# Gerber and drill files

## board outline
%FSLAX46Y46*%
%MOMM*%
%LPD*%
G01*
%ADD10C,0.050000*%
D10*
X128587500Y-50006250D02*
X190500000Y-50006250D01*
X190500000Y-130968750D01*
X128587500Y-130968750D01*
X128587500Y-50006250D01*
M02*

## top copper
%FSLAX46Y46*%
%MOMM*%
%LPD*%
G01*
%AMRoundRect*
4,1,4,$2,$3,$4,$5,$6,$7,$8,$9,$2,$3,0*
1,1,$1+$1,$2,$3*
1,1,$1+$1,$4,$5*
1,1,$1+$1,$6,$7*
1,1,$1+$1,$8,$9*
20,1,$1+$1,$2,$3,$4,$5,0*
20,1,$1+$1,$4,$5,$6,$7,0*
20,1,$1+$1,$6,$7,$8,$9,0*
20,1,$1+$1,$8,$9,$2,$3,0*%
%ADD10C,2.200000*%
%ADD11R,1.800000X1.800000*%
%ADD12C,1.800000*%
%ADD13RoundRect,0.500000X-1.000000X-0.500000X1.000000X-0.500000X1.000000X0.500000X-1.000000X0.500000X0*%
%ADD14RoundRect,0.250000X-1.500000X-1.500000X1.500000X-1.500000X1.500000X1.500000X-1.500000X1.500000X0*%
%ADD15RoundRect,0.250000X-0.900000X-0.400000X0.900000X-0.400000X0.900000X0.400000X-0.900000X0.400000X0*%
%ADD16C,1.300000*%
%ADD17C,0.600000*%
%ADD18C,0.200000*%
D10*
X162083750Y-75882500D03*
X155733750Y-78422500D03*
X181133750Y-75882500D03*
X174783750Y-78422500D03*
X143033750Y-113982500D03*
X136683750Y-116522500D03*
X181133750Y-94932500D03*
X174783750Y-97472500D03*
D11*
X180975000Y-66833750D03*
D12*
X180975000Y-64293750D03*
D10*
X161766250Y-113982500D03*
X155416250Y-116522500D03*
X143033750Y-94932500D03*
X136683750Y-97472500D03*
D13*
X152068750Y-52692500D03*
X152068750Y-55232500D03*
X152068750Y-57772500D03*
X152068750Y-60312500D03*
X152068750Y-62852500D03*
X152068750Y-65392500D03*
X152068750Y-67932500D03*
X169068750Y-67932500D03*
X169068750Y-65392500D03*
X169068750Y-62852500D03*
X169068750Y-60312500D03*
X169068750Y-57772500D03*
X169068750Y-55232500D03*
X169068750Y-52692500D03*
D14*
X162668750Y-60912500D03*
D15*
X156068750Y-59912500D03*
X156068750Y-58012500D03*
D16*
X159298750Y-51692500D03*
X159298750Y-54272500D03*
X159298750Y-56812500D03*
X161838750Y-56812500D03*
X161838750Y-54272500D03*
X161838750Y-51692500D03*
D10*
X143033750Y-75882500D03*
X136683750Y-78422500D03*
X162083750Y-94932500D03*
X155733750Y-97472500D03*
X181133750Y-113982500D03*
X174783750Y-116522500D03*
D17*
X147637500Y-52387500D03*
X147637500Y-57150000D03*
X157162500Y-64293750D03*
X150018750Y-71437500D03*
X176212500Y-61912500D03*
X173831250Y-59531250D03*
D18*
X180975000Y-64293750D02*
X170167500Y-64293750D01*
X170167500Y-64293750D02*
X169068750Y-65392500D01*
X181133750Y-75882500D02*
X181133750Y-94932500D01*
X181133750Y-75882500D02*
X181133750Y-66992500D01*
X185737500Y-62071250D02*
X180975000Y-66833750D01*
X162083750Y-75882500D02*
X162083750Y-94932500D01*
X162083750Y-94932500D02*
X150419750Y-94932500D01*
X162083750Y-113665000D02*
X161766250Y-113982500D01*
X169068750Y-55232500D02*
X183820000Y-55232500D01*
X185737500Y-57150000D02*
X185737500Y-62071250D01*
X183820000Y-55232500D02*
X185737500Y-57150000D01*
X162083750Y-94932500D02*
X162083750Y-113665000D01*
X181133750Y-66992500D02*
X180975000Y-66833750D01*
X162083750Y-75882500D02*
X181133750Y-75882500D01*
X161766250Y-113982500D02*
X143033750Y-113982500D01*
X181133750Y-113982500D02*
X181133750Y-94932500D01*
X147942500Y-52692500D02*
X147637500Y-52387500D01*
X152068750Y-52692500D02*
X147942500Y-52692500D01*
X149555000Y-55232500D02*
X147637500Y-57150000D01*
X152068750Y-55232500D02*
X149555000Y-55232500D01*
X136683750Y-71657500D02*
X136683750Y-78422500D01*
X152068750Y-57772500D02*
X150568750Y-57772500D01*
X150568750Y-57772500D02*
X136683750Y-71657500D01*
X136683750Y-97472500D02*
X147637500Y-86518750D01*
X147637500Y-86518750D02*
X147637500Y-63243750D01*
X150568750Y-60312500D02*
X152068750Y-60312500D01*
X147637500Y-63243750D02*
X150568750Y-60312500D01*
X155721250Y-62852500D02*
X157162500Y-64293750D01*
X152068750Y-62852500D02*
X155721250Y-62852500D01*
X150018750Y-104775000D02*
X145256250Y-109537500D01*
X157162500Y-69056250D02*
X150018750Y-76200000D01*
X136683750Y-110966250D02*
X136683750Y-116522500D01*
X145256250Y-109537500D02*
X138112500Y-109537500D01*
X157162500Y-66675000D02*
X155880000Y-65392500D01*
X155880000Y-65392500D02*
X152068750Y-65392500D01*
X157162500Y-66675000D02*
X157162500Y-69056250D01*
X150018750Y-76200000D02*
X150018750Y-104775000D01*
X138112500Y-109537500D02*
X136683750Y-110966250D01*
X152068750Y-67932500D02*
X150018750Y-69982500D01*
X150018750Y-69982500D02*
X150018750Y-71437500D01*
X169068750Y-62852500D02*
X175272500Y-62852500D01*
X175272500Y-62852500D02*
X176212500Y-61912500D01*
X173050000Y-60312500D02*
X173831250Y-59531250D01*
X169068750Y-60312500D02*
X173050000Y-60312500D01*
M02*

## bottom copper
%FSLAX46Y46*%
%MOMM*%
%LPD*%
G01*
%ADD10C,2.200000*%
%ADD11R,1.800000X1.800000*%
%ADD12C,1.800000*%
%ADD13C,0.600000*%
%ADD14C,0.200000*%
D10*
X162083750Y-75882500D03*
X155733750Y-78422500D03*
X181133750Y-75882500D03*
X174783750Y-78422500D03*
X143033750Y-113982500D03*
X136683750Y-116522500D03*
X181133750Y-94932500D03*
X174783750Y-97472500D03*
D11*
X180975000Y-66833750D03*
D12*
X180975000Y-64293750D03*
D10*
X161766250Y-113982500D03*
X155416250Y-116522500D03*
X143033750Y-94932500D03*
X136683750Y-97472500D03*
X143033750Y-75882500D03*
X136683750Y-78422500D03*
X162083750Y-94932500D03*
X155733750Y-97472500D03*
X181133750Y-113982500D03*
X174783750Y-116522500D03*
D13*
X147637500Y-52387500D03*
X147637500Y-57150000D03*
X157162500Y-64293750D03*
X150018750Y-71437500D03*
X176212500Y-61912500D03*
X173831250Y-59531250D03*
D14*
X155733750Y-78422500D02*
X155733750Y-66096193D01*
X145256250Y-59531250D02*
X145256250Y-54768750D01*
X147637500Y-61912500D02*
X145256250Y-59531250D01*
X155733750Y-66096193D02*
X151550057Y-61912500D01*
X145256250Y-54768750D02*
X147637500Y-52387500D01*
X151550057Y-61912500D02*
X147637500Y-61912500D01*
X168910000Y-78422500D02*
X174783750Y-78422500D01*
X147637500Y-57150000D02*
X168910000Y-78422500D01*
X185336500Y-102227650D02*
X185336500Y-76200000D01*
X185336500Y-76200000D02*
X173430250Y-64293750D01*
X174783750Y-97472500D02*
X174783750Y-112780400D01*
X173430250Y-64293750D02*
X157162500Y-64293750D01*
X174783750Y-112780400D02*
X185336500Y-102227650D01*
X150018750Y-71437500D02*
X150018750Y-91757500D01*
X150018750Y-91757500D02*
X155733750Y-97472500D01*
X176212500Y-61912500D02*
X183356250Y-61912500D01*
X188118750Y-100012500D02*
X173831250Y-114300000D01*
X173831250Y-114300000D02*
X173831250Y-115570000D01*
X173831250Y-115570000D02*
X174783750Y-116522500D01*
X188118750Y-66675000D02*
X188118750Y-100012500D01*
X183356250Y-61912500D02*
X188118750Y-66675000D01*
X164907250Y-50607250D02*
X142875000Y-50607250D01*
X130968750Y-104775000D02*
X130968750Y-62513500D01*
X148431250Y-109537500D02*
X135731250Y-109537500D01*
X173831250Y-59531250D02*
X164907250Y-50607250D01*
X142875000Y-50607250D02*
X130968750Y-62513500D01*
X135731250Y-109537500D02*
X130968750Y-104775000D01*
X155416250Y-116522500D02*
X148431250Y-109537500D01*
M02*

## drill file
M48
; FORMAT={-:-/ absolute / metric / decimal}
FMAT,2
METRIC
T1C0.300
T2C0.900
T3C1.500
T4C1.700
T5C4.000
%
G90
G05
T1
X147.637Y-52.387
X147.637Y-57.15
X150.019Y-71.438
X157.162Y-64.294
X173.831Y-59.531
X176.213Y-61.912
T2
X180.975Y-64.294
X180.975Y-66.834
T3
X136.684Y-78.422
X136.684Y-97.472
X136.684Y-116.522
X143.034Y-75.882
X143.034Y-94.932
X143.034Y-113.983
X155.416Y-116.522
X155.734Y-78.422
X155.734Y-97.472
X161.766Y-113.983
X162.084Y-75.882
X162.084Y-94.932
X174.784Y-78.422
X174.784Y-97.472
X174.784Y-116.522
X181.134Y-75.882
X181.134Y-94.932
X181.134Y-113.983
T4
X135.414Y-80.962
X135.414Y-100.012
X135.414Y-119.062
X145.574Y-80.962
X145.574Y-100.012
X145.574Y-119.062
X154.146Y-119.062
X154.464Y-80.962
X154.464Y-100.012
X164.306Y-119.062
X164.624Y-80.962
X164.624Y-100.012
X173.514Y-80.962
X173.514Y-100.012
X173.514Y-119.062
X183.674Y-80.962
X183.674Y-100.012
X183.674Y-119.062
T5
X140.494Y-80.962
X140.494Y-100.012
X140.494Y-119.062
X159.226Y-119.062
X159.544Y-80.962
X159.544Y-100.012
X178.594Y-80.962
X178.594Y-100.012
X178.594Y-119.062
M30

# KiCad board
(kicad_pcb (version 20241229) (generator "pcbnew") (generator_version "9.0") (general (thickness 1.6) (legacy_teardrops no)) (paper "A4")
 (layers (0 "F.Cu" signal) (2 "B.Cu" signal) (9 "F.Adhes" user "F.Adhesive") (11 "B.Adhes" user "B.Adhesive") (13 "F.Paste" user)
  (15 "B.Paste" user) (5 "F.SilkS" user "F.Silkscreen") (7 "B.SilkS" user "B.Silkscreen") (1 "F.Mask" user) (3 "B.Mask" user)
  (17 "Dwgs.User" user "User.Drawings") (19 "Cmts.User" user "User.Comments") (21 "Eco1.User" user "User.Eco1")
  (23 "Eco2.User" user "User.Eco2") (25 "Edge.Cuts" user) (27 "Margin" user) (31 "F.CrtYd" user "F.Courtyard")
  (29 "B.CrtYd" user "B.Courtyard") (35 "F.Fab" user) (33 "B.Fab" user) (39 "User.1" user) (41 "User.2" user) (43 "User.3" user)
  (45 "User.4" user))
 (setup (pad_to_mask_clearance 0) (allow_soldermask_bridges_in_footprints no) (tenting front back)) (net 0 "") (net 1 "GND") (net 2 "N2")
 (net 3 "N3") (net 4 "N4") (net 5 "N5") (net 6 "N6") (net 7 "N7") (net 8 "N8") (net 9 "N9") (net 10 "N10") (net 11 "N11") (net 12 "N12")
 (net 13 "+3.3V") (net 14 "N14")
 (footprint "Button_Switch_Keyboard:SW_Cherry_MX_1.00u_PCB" (layer "F.Cu") (at 162.08375 75.8825)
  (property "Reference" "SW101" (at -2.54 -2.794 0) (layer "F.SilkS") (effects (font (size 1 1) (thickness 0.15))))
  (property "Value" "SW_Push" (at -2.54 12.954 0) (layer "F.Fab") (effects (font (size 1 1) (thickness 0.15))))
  (pad "" np_thru_hole circle (at -7.62 5.08) (size 1.7 1.7) (drill 1.7) (layers "*.Cu" "*.Mask"))
  (pad "" np_thru_hole circle (at -2.54 5.08) (size 4 4) (drill 4) (layers "*.Cu" "*.Mask"))
  (pad "" np_thru_hole circle (at 2.54 5.08) (size 1.7 1.7) (drill 1.7) (layers "*.Cu" "*.Mask"))
  (pad "1" thru_hole circle (at 0 0) (size 2.2 2.2) (drill 1.5) (layers "*.Cu" "*.Mask") (remove_unused_layers no) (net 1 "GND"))
  (pad "2" thru_hole circle (at -6.35 2.54) (size 2.2 2.2) (drill 1.5) (layers "*.Cu" "*.Mask") (remove_unused_layers no) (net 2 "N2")))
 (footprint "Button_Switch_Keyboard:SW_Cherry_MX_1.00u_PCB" (layer "F.Cu") (at 181.13375 75.8825)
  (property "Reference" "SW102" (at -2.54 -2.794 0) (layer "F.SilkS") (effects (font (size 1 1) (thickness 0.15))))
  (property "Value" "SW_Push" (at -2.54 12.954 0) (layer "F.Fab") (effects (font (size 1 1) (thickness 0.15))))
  (pad "" np_thru_hole circle (at -7.62 5.08) (size 1.7 1.7) (drill 1.7) (layers "*.Cu" "*.Mask"))
  (pad "" np_thru_hole circle (at -2.54 5.08) (size 4 4) (drill 4) (layers "*.Cu" "*.Mask"))
  (pad "" np_thru_hole circle (at 2.54 5.08) (size 1.7 1.7) (drill 1.7) (layers "*.Cu" "*.Mask"))
  (pad "1" thru_hole circle (at 0 0) (size 2.2 2.2) (drill 1.5) (layers "*.Cu" "*.Mask") (remove_unused_layers no) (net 1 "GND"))
  (pad "2" thru_hole circle (at -6.35 2.54) (size 2.2 2.2) (drill 1.5) (layers "*.Cu" "*.Mask") (remove_unused_layers no) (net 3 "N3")))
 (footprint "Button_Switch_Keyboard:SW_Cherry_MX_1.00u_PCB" (layer "F.Cu") (at 143.03375 113.9825)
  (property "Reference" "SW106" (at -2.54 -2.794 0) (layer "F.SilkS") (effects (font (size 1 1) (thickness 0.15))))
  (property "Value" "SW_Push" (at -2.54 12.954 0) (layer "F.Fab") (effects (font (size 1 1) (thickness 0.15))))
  (pad "" np_thru_hole circle (at -7.62 5.08) (size 1.7 1.7) (drill 1.7) (layers "*.Cu" "*.Mask"))
  (pad "" np_thru_hole circle (at -2.54 5.08) (size 4 4) (drill 4) (layers "*.Cu" "*.Mask"))
  (pad "" np_thru_hole circle (at 2.54 5.08) (size 1.7 1.7) (drill 1.7) (layers "*.Cu" "*.Mask"))
  (pad "1" thru_hole circle (at 0 0) (size 2.2 2.2) (drill 1.5) (layers "*.Cu" "*.Mask") (remove_unused_layers no) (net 1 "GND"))
  (pad "2" thru_hole circle (at -6.35 2.54) (size 2.2 2.2) (drill 1.5) (layers "*.Cu" "*.Mask") (remove_unused_layers no) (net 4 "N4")))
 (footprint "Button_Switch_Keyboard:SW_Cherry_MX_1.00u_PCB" (layer "F.Cu") (at 181.13375 94.9325)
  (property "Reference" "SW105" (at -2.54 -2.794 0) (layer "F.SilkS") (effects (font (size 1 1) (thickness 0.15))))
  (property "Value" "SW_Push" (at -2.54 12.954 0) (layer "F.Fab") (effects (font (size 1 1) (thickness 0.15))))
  (pad "" np_thru_hole circle (at -7.62 5.08) (size 1.7 1.7) (drill 1.7) (layers "*.Cu" "*.Mask"))
  (pad "" np_thru_hole circle (at -2.54 5.08) (size 4 4) (drill 4) (layers "*.Cu" "*.Mask"))
  (pad "" np_thru_hole circle (at 2.54 5.08) (size 1.7 1.7) (drill 1.7) (layers "*.Cu" "*.Mask"))
  (pad "1" thru_hole circle (at 0 0) (size 2.2 2.2) (drill 1.5) (layers "*.Cu" "*.Mask") (remove_unused_layers no) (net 1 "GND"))
  (pad "2" thru_hole circle (at -6.35 2.54) (size 2.2 2.2) (drill 1.5) (layers "*.Cu" "*.Mask") (remove_unused_layers no) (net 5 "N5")))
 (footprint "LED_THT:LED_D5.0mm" (layer "F.Cu") (at 180.975 66.83375 90)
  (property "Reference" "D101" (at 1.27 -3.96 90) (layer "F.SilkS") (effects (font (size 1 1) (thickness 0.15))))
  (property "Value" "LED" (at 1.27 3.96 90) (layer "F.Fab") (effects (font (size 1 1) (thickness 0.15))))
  (pad "1" thru_hole rect (at 0 0 90) (size 1.8 1.8) (drill 0.9) (layers "*.Cu" "*.Mask") (remove_unused_layers no) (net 1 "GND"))
  (pad "2" thru_hole circle (at 2.54 0 90) (size 1.8 1.8) (drill 0.9) (layers "*.Cu" "*.Mask") (remove_unused_layers no) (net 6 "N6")))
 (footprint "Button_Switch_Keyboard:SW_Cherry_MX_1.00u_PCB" (layer "F.Cu") (at 161.76625 113.9825)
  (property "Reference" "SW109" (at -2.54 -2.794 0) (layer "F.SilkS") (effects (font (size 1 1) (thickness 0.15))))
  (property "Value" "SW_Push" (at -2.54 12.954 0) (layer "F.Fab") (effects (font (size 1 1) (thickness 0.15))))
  (pad "" np_thru_hole circle (at -7.62 5.08) (size 1.7 1.7) (drill 1.7) (layers "*.Cu" "*.Mask"))
  (pad "" np_thru_hole circle (at -2.54 5.08) (size 4 4) (drill 4) (layers "*.Cu" "*.Mask"))
  (pad "" np_thru_hole circle (at 2.54 5.08) (size 1.7 1.7) (drill 1.7) (layers "*.Cu" "*.Mask"))
  (pad "1" thru_hole circle (at 0 0) (size 2.2 2.2) (drill 1.5) (layers "*.Cu" "*.Mask") (remove_unused_layers no) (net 1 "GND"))
  (pad "2" thru_hole circle (at -6.35 2.54) (size 2.2 2.2) (drill 1.5) (layers "*.Cu" "*.Mask") (remove_unused_layers no) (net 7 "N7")))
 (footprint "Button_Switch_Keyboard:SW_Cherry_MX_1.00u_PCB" (layer "F.Cu") (at 143.03375 94.9325)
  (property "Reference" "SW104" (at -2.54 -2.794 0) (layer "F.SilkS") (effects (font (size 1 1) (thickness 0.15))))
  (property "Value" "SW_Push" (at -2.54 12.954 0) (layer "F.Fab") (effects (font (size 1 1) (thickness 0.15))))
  (pad "" np_thru_hole circle (at -7.62 5.08) (size 1.7 1.7) (drill 1.7) (layers "*.Cu" "*.Mask"))
  (pad "" np_thru_hole circle (at -2.54 5.08) (size 4 4) (drill 4) (layers "*.Cu" "*.Mask"))
  (pad "" np_thru_hole circle (at 2.54 5.08) (size 1.7 1.7) (drill 1.7) (layers "*.Cu" "*.Mask"))
  (pad "1" thru_hole circle (at 0 0) (size 2.2 2.2) (drill 1.5) (layers "*.Cu" "*.Mask") (remove_unused_layers no) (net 1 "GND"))
  (pad "2" thru_hole circle (at -6.35 2.54) (size 2.2 2.2) (drill 1.5) (layers "*.Cu" "*.Mask") (remove_unused_layers no) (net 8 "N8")))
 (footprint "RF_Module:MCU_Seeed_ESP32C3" (layer "F.Cu") (at 160.56875 60.3125)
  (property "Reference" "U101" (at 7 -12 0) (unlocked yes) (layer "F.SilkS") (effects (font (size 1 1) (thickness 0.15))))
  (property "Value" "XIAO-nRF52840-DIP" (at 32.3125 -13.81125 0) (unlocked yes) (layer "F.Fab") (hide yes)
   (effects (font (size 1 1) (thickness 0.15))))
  (pad "" smd roundrect (at 1.1 -0.4) (size 1.5 1.5) (layers "F.Paste") (roundrect_rratio 0.1666666667))
  (pad "" smd roundrect (at 1.1 1.6) (size 1.5 1.5) (layers "F.Paste") (roundrect_rratio 0.1666666667))
  (pad "" smd roundrect (at 3.1 -0.4) (size 1.5 1.5) (layers "F.Paste") (roundrect_rratio 0.1666666667))
  (pad "" smd roundrect (at 3.1 1.6) (size 1.5 1.5) (layers "F.Paste") (roundrect_rratio 0.1666666667))
  (pad "1" smd roundrect (at -8.5 -7.62) (size 3 2) (layers "F.Cu" "F.Mask" "F.Paste") (roundrect_rratio 0.25) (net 2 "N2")
   (thermal_bridge_angle 45))
  (pad "2" smd roundrect (at -8.5 -5.08) (size 3 2) (layers "F.Cu" "F.Mask" "F.Paste") (roundrect_rratio 0.25) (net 3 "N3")
   (thermal_bridge_angle 45))
  (pad "3" smd roundrect (at -8.5 -2.54) (size 3 2) (layers "F.Cu" "F.Mask" "F.Paste") (roundrect_rratio 0.25) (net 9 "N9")
   (thermal_bridge_angle 45))
  (pad "4" smd roundrect (at -8.5 0) (size 3 2) (layers "F.Cu" "F.Mask" "F.Paste") (roundrect_rratio 0.25) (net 8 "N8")
   (thermal_bridge_angle 45))
  (pad "5" smd roundrect (at -8.5 2.54) (size 3 2) (layers "F.Cu" "F.Mask" "F.Paste") (roundrect_rratio 0.25) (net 5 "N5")
   (thermal_bridge_angle 45))
  (pad "6" smd roundrect (at -8.5 5.08) (size 3 2) (layers "F.Cu" "F.Mask" "F.Paste") (roundrect_rratio 0.25) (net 4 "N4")
   (thermal_bridge_angle 45))
  (pad "7" smd roundrect (at -8.5 7.62) (size 3 2) (layers "F.Cu" "F.Mask" "F.Paste") (roundrect_rratio 0.25) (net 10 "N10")
   (thermal_bridge_angle 45))
  (pad "8" smd roundrect (at 8.5 7.62) (size 3 2) (layers "F.Cu" "F.Mask" "F.Paste") (roundrect_rratio 0.25) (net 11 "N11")
   (thermal_bridge_angle 45))
  (pad "9" smd roundrect (at 8.5 5.08) (size 3 2) (layers "F.Cu" "F.Mask" "F.Paste") (roundrect_rratio 0.25) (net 6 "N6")
   (thermal_bridge_angle 45))
  (pad "10" smd roundrect (at 8.5 2.54) (size 3 2) (layers "F.Cu" "F.Mask" "F.Paste") (roundrect_rratio 0.25) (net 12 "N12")
   (thermal_bridge_angle 45))
  (pad "11" smd roundrect (at 8.5 0) (size 3 2) (layers "F.Cu" "F.Mask" "F.Paste") (roundrect_rratio 0.25) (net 7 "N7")
   (thermal_bridge_angle 45))
  (pad "12" smd roundrect (at 8.5 -2.54) (size 3 2) (layers "F.Cu" "F.Mask" "F.Paste") (roundrect_rratio 0.25) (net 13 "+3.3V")
   (thermal_bridge_angle 45))
  (pad "13" smd roundrect (at 8.5 -5.08) (size 3 2) (layers "F.Cu" "F.Mask" "F.Paste") (roundrect_rratio 0.25) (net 1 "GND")
   (thermal_bridge_angle 45))
  (pad "14" smd roundrect (at 8.5 -7.62) (size 3 2) (layers "F.Cu" "F.Mask" "F.Paste") (roundrect_rratio 0.25) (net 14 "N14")
   (thermal_bridge_angle 45))
  (pad "15" smd roundrect (at 2.1 0.6) (size 3.5 3.5) (layers "F.Cu" "F.Mask") (roundrect_rratio 0.07142857143))
  (pad "16" smd roundrect (at -4.5 -0.4) (size 2.3 1.3) (layers "F.Cu" "F.Mask" "F.Paste") (roundrect_rratio 0.1923076923))
  (pad "17" smd roundrect (at -4.5 -2.3) (size 2.3 1.3) (layers "F.Cu" "F.Mask" "F.Paste") (roundrect_rratio 0.1923076923))
  (pad "18" smd circle (at -1.27 -8.62) (size 1.3 1.3) (layers "F.Cu" "F.Mask" "F.Paste"))
  (pad "19" smd circle (at -1.27 -6.04) (size 1.3 1.3) (layers "F.Cu" "F.Mask" "F.Paste"))
  (pad "20" smd circle (at -1.27 -3.5) (size 1.3 1.3) (layers "F.Cu" "F.Mask" "F.Paste"))
  (pad "21" smd circle (at 1.27 -3.5) (size 1.3 1.3) (layers "F.Cu" "F.Mask" "F.Paste"))
  (pad "22" smd circle (at 1.27 -6.04) (size 1.3 1.3) (layers "F.Cu" "F.Mask" "F.Paste"))
  (pad "23" smd circle (at 1.27 -8.62) (size 1.3 1.3) (layers "F.Cu" "F.Mask" "F.Paste")))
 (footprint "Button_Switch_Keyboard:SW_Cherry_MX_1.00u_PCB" (layer "F.Cu") (at 143.03375 75.8825)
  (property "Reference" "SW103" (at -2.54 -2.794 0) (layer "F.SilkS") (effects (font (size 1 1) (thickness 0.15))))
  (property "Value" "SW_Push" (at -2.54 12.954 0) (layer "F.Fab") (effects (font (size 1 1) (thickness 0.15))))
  (pad "" np_thru_hole circle (at -7.62 5.08) (size 1.7 1.7) (drill 1.7) (layers "*.Cu" "*.Mask"))
  (pad "" np_thru_hole circle (at -2.54 5.08) (size 4 4) (drill 4) (layers "*.Cu" "*.Mask"))
  (pad "" np_thru_hole circle (at 2.54 5.08) (size 1.7 1.7) (drill 1.7) (layers "*.Cu" "*.Mask"))
  (pad "1" thru_hole circle (at 0 0) (size 2.2 2.2) (drill 1.5) (layers "*.Cu" "*.Mask") (remove_unused_layers no) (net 1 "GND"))
  (pad "2" thru_hole circle (at -6.35 2.54) (size 2.2 2.2) (drill 1.5) (layers "*.Cu" "*.Mask") (remove_unused_layers no) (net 9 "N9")))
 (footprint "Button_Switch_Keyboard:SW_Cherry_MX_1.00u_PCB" (layer "F.Cu") (at 162.08375 94.9325)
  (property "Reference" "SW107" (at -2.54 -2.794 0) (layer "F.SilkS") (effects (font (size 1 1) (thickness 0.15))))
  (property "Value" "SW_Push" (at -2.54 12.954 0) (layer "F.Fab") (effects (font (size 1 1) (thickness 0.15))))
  (pad "" np_thru_hole circle (at -7.62 5.08) (size 1.7 1.7) (drill 1.7) (layers "*.Cu" "*.Mask"))
  (pad "" np_thru_hole circle (at -2.54 5.08) (size 4 4) (drill 4) (layers "*.Cu" "*.Mask"))
  (pad "" np_thru_hole circle (at 2.54 5.08) (size 1.7 1.7) (drill 1.7) (layers "*.Cu" "*.Mask"))
  (pad "1" thru_hole circle (at 0 0) (size 2.2 2.2) (drill 1.5) (layers "*.Cu" "*.Mask") (remove_unused_layers no) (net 1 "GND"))
  (pad "2" thru_hole circle (at -6.35 2.54) (size 2.2 2.2) (drill 1.5) (layers "*.Cu" "*.Mask") (remove_unused_layers no) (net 10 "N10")))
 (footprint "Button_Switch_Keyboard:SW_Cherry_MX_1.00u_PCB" (layer "F.Cu") (at 181.13375 113.9825)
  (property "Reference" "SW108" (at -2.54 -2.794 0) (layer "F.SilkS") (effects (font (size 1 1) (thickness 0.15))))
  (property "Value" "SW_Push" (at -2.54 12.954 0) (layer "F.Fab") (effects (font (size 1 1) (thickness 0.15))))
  (pad "" np_thru_hole circle (at -7.62 5.08) (size 1.7 1.7) (drill 1.7) (layers "*.Cu" "*.Mask"))
  (pad "" np_thru_hole circle (at -2.54 5.08) (size 4 4) (drill 4) (layers "*.Cu" "*.Mask"))
  (pad "" np_thru_hole circle (at 2.54 5.08) (size 1.7 1.7) (drill 1.7) (layers "*.Cu" "*.Mask"))
  (pad "1" thru_hole circle (at 0 0) (size 2.2 2.2) (drill 1.5) (layers "*.Cu" "*.Mask") (remove_unused_layers no) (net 1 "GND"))
  (pad "2" thru_hole circle (at -6.35 2.54) (size 2.2 2.2) (drill 1.5) (layers "*.Cu" "*.Mask") (remove_unused_layers no) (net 12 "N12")))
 (gr_rect (start 128.5875 50.00625) (end 190.5 130.96875) (stroke (width 0.05) (type default)) (fill no) (layer "Edge.Cuts"))
 (segment (start 180.975 64.29375) (end 170.1675 64.29375) (width 0.2) (layer "F.Cu") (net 6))
 (segment (start 170.1675 64.29375) (end 169.06875 65.3925) (width 0.2) (layer "F.Cu") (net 6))
 (segment (start 181.13375 75.8825) (end 181.13375 94.9325) (width 0.2) (layer "F.Cu") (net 1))
 (segment (start 181.13375 75.8825) (end 181.13375 66.9925) (width 0.2) (layer "F.Cu") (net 1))
 (segment (start 185.7375 62.07125) (end 180.975 66.83375) (width 0.2) (layer "F.Cu") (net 1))
 (segment (start 162.08375 75.8825) (end 162.08375 94.9325) (width 0.2) (layer "F.Cu") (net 1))
 (segment (start 162.08375 94.9325) (end 150.41975 94.9325) (width 0.2) (layer "F.Cu") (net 1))
 (segment (start 162.08375 113.665) (end 161.76625 113.9825) (width 0.2) (layer "F.Cu") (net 1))
 (segment (start 169.06875 55.2325) (end 183.82 55.2325) (width 0.2) (layer "F.Cu") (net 1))
 (segment (start 185.7375 57.15) (end 185.7375 62.07125) (width 0.2) (layer "F.Cu") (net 1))
 (segment (start 183.82 55.2325) (end 185.7375 57.15) (width 0.2) (layer "F.Cu") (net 1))
 (segment (start 162.08375 94.9325) (end 162.08375 113.665) (width 0.2) (layer "F.Cu") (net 1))
 (segment (start 181.13375 66.9925) (end 180.975 66.83375) (width 0.2) (layer "F.Cu") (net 1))
 (segment (start 162.08375 75.8825) (end 181.13375 75.8825) (width 0.2) (layer "F.Cu") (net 1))
 (segment (start 161.76625 113.9825) (end 143.03375 113.9825) (width 0.2) (layer "F.Cu") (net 1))
 (segment (start 181.13375 113.9825) (end 181.13375 94.9325) (width 0.2) (layer "F.Cu") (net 1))
 (segment (start 147.9425 52.6925) (end 147.6375 52.3875) (width 0.2) (layer "F.Cu") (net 2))
 (segment (start 152.06875 52.6925) (end 147.9425 52.6925) (width 0.2) (layer "F.Cu") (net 2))
 (via (at 147.6375 52.3875) (size 0.6) (drill 0.3) (layers "F.Cu" "B.Cu") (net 2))
 (segment (start 155.73375 78.4225) (end 155.73375 66.096193) (width 0.2) (layer "B.Cu") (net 2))
 (segment (start 145.25625 59.53125) (end 145.25625 54.76875) (width 0.2) (layer "B.Cu") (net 2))
 (segment (start 147.6375 61.9125) (end 145.25625 59.53125) (width 0.2) (layer "B.Cu") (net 2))
 (segment (start 155.73375 66.096193) (end 151.550057 61.9125) (width 0.2) (layer "B.Cu") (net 2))
 (segment (start 145.25625 54.76875) (end 147.6375 52.3875) (width 0.2) (layer "B.Cu") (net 2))
 (segment (start 151.550057 61.9125) (end 147.6375 61.9125) (width 0.2) (layer "B.Cu") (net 2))
 (segment (start 149.555 55.2325) (end 147.6375 57.15) (width 0.2) (layer "F.Cu") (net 3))
 (segment (start 152.06875 55.2325) (end 149.555 55.2325) (width 0.2) (layer "F.Cu") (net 3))
 (via (at 147.6375 57.15) (size 0.6) (drill 0.3) (layers "F.Cu" "B.Cu") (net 3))
 (segment (start 168.91 78.4225) (end 174.78375 78.4225) (width 0.2) (layer "B.Cu") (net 3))
 (segment (start 147.6375 57.15) (end 168.91 78.4225) (width 0.2) (layer "B.Cu") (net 3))
 (segment (start 136.68375 71.6575) (end 136.68375 78.4225) (width 0.2) (layer "F.Cu") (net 9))
 (segment (start 152.06875 57.7725) (end 150.56875 57.7725) (width 0.2) (layer "F.Cu") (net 9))
 (segment (start 150.56875 57.7725) (end 136.68375 71.6575) (width 0.2) (layer "F.Cu") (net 9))
 (segment (start 136.68375 97.4725) (end 147.6375 86.51875) (width 0.2) (layer "F.Cu") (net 8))
 (segment (start 147.6375 86.51875) (end 147.6375 63.24375) (width 0.2) (layer "F.Cu") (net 8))
 (segment (start 150.56875 60.3125) (end 152.06875 60.3125) (width 0.2) (layer "F.Cu") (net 8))
 (segment (start 147.6375 63.24375) (end 150.56875 60.3125) (width 0.2) (layer "F.Cu") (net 8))
 (segment (start 155.72125 62.8525) (end 157.1625 64.29375) (width 0.2) (layer "F.Cu") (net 5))
 (segment (start 152.06875 62.8525) (end 155.72125 62.8525) (width 0.2) (layer "F.Cu") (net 5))
 (via (at 157.1625 64.29375) (size 0.6) (drill 0.3) (layers "F.Cu" "B.Cu") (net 5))
 (segment (start 185.3365 102.22765) (end 185.3365 76.2) (width 0.2) (layer "B.Cu") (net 5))
 (segment (start 185.3365 76.2) (end 173.43025 64.29375) (width 0.2) (layer "B.Cu") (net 5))
 (segment (start 174.78375 97.4725) (end 174.78375 112.7804) (width 0.2) (layer "B.Cu") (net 5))
 (segment (start 173.43025 64.29375) (end 157.1625 64.29375) (width 0.2) (layer "B.Cu") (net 5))
 (segment (start 174.78375 112.7804) (end 185.3365 102.22765) (width 0.2) (layer "B.Cu") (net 5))
 (segment (start 150.01875 104.775) (end 145.25625 109.5375) (width 0.2) (layer "F.Cu") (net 4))
 (segment (start 157.1625 69.05625) (end 150.01875 76.2) (width 0.2) (layer "F.Cu") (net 4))
 (segment (start 136.68375 110.96625) (end 136.68375 116.5225) (width 0.2) (layer "F.Cu") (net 4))
 (segment (start 145.25625 109.5375) (end 138.1125 109.5375) (width 0.2) (layer "F.Cu") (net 4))
 (segment (start 157.1625 66.675) (end 155.88 65.3925) (width 0.2) (layer "F.Cu") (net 4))
 (segment (start 155.88 65.3925) (end 152.06875 65.3925) (width 0.2) (layer "F.Cu") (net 4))
 (segment (start 157.1625 66.675) (end 157.1625 69.05625) (width 0.2) (layer "F.Cu") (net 4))
 (segment (start 150.01875 76.2) (end 150.01875 104.775) (width 0.2) (layer "F.Cu") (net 4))
 (segment (start 138.1125 109.5375) (end 136.68375 110.96625) (width 0.2) (layer "F.Cu") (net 4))
 (segment (start 152.06875 67.9325) (end 150.01875 69.9825) (width 0.2) (layer "F.Cu") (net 10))
 (segment (start 150.01875 69.9825) (end 150.01875 71.4375) (width 0.2) (layer "F.Cu") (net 10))
 (via (at 150.01875 71.4375) (size 0.6) (drill 0.3) (layers "F.Cu" "B.Cu") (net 10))
 (segment (start 150.01875 71.4375) (end 150.01875 91.7575) (width 0.2) (layer "B.Cu") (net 10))
 (segment (start 150.01875 91.7575) (end 155.73375 97.4725) (width 0.2) (layer "B.Cu") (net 10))
 (segment (start 169.06875 62.8525) (end 175.2725 62.8525) (width 0.2) (layer "F.Cu") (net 12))
 (segment (start 175.2725 62.8525) (end 176.2125 61.9125) (width 0.2) (layer "F.Cu") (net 12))
 (via (at 176.2125 61.9125) (size 0.6) (drill 0.3) (layers "F.Cu" "B.Cu") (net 12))
 (segment (start 176.2125 61.9125) (end 183.35625 61.9125) (width 0.2) (layer "B.Cu") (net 12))
 (segment (start 188.11875 100.0125) (end 173.83125 114.3) (width 0.2) (layer "B.Cu") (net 12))
 (segment (start 173.83125 114.3) (end 173.83125 115.57) (width 0.2) (layer "B.Cu") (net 12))
 (segment (start 173.83125 115.57) (end 174.78375 116.5225) (width 0.2) (layer "B.Cu") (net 12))
 (segment (start 188.11875 66.675) (end 188.11875 100.0125) (width 0.2) (layer "B.Cu") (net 12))
 (segment (start 183.35625 61.9125) (end 188.11875 66.675) (width 0.2) (layer "B.Cu") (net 12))
 (segment (start 173.05 60.3125) (end 173.83125 59.53125) (width 0.2) (layer "F.Cu") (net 7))
 (segment (start 169.06875 60.3125) (end 173.05 60.3125) (width 0.2) (layer "F.Cu") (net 7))
 (via (at 173.83125 59.53125) (size 0.6) (drill 0.3) (layers "F.Cu" "B.Cu") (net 7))
 (segment (start 164.90725 50.60725) (end 142.875 50.60725) (width 0.2) (layer "B.Cu") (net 7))
 (segment (start 130.96875 104.775) (end 130.96875 62.5135) (width 0.2) (layer "B.Cu") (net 7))
 (segment (start 148.43125 109.5375) (end 135.73125 109.5375) (width 0.2) (layer "B.Cu") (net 7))
 (segment (start 173.83125 59.53125) (end 164.90725 50.60725) (width 0.2) (layer "B.Cu") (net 7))
 (segment (start 142.875 50.60725) (end 130.96875 62.5135) (width 0.2) (layer "B.Cu") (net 7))
 (segment (start 135.73125 109.5375) (end 130.96875 104.775) (width 0.2) (layer "B.Cu") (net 7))
 (segment (start 155.41625 116.5225) (end 148.43125 109.5375) (width 0.2) (layer "B.Cu") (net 7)))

